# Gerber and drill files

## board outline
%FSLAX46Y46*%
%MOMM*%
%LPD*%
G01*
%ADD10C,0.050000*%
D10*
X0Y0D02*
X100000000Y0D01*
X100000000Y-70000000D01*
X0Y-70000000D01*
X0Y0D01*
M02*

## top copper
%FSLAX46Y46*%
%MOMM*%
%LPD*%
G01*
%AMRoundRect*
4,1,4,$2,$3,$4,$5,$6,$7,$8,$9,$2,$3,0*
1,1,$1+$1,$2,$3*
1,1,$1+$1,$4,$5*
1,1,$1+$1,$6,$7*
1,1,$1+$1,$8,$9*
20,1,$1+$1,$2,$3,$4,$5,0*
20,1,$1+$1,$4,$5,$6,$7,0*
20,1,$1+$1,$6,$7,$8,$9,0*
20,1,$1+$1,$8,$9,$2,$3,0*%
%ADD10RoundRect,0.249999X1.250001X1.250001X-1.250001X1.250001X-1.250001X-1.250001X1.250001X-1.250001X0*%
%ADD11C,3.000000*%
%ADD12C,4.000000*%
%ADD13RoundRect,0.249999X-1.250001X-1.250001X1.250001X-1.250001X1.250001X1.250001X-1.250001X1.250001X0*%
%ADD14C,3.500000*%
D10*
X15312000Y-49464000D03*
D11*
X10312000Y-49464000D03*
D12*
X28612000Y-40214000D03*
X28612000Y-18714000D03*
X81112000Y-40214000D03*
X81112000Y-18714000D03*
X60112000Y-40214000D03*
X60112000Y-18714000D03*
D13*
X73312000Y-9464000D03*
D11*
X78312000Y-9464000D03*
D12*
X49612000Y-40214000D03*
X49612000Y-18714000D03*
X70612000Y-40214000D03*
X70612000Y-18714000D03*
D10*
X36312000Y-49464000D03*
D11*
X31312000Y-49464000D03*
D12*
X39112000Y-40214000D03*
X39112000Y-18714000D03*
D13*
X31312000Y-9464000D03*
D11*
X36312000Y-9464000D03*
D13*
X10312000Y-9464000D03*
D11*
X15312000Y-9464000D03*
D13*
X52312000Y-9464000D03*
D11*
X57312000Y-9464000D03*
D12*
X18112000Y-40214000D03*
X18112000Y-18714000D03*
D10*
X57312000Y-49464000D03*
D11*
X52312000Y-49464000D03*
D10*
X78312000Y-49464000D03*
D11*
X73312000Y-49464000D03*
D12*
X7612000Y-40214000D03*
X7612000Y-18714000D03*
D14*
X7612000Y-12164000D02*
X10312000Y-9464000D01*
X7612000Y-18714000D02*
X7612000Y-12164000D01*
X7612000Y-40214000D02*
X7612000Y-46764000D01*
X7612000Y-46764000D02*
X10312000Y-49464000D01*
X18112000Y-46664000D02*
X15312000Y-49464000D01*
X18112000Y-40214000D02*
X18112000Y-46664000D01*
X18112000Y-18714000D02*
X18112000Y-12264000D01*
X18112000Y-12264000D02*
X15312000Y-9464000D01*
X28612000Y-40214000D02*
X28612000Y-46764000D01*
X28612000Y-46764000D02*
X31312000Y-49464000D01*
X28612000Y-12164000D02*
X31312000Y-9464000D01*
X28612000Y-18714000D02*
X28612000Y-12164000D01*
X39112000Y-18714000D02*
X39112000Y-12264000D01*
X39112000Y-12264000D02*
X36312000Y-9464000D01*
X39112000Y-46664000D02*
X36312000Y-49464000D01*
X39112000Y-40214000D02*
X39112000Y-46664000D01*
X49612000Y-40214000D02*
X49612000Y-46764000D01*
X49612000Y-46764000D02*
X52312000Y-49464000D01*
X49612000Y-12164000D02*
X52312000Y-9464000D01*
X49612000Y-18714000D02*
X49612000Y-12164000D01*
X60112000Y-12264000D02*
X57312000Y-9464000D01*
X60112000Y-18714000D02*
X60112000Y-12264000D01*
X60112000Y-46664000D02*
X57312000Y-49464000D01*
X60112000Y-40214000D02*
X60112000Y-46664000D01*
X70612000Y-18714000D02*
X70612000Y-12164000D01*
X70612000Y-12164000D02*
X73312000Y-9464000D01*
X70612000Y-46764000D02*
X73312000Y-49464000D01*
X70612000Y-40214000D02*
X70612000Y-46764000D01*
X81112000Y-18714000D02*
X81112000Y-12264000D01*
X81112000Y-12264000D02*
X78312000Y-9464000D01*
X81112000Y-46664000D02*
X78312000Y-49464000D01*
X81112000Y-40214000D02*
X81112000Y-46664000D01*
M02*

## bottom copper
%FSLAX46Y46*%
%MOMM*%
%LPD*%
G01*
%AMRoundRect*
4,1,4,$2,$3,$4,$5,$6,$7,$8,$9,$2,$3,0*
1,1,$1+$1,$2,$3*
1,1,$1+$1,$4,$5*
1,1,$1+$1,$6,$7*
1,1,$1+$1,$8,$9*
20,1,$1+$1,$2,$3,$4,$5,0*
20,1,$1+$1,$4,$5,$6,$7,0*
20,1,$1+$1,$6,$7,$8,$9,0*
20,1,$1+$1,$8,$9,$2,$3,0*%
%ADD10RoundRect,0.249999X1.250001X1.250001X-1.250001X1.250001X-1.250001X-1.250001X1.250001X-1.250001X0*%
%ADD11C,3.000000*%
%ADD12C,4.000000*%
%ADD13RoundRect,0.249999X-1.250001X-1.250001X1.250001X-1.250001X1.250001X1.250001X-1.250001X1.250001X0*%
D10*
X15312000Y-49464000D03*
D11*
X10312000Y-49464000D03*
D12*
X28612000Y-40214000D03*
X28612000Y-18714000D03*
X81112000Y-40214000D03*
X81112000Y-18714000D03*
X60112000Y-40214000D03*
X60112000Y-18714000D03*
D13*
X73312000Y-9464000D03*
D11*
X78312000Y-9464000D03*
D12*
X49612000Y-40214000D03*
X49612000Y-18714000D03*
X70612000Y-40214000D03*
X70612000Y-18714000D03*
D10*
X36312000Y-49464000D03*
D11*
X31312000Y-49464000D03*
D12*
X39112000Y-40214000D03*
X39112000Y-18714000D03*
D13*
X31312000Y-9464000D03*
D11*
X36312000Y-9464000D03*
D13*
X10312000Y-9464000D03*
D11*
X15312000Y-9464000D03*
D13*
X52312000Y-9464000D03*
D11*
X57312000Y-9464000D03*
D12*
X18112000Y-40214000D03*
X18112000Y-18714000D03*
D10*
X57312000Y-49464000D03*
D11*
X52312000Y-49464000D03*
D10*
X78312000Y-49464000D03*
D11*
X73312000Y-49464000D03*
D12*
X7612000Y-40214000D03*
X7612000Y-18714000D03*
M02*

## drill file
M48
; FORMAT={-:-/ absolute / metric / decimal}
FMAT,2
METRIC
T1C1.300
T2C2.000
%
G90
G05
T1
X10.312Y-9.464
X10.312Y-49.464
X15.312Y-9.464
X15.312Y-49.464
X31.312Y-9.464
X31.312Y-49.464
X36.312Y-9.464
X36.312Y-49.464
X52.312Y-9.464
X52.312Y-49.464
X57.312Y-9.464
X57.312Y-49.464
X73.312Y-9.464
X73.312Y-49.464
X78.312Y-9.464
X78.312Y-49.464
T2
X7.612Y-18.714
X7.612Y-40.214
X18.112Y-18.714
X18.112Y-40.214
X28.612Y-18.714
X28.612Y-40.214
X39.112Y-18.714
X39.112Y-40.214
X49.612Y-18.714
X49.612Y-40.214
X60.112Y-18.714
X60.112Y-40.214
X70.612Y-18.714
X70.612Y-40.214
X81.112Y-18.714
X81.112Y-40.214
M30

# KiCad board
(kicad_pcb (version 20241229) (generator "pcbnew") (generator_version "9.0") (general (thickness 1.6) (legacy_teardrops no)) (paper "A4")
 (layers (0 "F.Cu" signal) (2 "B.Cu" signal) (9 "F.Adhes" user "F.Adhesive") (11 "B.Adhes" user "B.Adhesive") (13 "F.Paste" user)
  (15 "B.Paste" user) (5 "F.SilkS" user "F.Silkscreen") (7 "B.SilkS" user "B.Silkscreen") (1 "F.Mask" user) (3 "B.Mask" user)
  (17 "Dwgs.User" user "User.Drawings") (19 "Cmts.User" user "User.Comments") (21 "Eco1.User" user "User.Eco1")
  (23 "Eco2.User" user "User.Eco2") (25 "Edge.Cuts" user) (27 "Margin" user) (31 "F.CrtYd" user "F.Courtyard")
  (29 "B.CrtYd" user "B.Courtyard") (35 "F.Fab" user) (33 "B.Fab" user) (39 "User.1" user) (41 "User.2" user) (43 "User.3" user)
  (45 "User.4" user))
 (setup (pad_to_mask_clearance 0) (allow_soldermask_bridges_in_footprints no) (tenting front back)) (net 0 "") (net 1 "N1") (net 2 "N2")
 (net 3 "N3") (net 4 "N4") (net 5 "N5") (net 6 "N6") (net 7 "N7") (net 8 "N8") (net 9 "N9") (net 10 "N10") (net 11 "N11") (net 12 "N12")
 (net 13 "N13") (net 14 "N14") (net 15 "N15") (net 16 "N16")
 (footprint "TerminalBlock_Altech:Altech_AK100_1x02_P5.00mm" (layer "F.Cu") (at 15.312 49.464 180)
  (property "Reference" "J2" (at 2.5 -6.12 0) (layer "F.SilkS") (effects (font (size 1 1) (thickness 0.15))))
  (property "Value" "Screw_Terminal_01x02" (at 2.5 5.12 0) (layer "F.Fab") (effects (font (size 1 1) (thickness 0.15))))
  (pad "1" thru_hole roundrect (at 0 0 180) (size 3 3) (drill 1.3) (layers "*.Cu" "*.Mask") (remove_unused_layers no)
   (roundrect_rratio 0.083333) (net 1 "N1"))
  (pad "2" thru_hole circle (at 5 0 180) (size 3 3) (drill 1.3) (layers "*.Cu" "*.Mask") (remove_unused_layers no) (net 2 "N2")))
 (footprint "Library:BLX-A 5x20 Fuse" (layer "F.Cu") (at 28.612 29.464 90)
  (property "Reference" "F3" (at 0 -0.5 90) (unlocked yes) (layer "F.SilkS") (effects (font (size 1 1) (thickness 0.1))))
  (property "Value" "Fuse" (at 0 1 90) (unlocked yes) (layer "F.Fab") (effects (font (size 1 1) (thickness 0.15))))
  (pad "1" thru_hole circle (at -10.75 0 90) (size 4 4) (drill 2) (layers "*.Cu" "*.Mask") (remove_unused_layers no) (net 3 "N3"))
  (pad "2" thru_hole circle (at 10.75 0 90) (size 4 4) (drill 2) (layers "*.Cu" "*.Mask") (remove_unused_layers no) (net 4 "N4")))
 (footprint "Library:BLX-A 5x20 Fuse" (layer "F.Cu") (at 81.112 29.464 90)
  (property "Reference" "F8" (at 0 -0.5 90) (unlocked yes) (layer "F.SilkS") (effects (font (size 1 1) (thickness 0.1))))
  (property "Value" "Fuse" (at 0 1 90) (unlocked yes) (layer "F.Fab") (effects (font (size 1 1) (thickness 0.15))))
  (pad "1" thru_hole circle (at -10.75 0 90) (size 4 4) (drill 2) (layers "*.Cu" "*.Mask") (remove_unused_layers no) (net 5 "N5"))
  (pad "2" thru_hole circle (at 10.75 0 90) (size 4 4) (drill 2) (layers "*.Cu" "*.Mask") (remove_unused_layers no) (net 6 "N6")))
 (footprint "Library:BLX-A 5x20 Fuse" (layer "F.Cu") (at 60.112 29.464 90)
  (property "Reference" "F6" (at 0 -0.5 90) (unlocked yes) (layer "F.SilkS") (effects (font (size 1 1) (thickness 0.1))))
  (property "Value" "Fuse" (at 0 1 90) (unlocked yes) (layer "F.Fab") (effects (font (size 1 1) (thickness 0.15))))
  (pad "1" thru_hole circle (at -10.75 0 90) (size 4 4) (drill 2) (layers "*.Cu" "*.Mask") (remove_unused_layers no) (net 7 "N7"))
  (pad "2" thru_hole circle (at 10.75 0 90) (size 4 4) (drill 2) (layers "*.Cu" "*.Mask") (remove_unused_layers no) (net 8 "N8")))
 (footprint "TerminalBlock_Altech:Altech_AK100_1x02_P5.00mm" (layer "F.Cu") (at 73.312 9.464)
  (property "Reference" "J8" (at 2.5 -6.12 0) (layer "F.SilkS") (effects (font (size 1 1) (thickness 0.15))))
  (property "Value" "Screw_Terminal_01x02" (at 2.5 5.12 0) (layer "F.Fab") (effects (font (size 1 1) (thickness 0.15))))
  (pad "1" thru_hole roundrect (at 0 0) (size 3 3) (drill 1.3) (layers "*.Cu" "*.Mask") (remove_unused_layers no)
   (roundrect_rratio 0.083333) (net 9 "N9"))
  (pad "2" thru_hole circle (at 5 0) (size 3 3) (drill 1.3) (layers "*.Cu" "*.Mask") (remove_unused_layers no) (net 6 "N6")))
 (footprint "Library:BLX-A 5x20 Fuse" (layer "F.Cu") (at 49.612 29.464 90)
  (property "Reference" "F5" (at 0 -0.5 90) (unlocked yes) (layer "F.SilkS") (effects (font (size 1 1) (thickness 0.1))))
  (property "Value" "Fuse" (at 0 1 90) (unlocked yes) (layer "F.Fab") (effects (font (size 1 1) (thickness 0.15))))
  (pad "1" thru_hole circle (at -10.75 0 90) (size 4 4) (drill 2) (layers "*.Cu" "*.Mask") (remove_unused_layers no) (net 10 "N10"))
  (pad "2" thru_hole circle (at 10.75 0 90) (size 4 4) (drill 2) (layers "*.Cu" "*.Mask") (remove_unused_layers no) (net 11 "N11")))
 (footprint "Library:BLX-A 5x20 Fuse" (layer "F.Cu") (at 70.612 29.464 90)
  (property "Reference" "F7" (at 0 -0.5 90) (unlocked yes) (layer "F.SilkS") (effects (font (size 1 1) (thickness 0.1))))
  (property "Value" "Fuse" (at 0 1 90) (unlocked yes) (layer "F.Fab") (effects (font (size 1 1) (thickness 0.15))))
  (pad "1" thru_hole circle (at -10.75 0 90) (size 4 4) (drill 2) (layers "*.Cu" "*.Mask") (remove_unused_layers no) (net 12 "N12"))
  (pad "2" thru_hole circle (at 10.75 0 90) (size 4 4) (drill 2) (layers "*.Cu" "*.Mask") (remove_unused_layers no) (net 9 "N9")))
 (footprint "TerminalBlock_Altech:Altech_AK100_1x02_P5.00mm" (layer "F.Cu") (at 36.312 49.464 180)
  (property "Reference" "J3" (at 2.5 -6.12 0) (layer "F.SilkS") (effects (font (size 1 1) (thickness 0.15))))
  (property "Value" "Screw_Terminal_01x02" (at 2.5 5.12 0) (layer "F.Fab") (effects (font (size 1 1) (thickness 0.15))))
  (pad "1" thru_hole roundrect (at 0 0 180) (size 3 3) (drill 1.3) (layers "*.Cu" "*.Mask") (remove_unused_layers no)
   (roundrect_rratio 0.083333) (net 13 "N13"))
  (pad "2" thru_hole circle (at 5 0 180) (size 3 3) (drill 1.3) (layers "*.Cu" "*.Mask") (remove_unused_layers no) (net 3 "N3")))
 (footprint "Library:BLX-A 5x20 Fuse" (layer "F.Cu") (at 39.112 29.464 90)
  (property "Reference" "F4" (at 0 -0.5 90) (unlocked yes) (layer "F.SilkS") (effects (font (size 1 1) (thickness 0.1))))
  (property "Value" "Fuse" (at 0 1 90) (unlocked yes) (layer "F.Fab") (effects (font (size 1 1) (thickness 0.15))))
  (pad "1" thru_hole circle (at -10.75 0 90) (size 4 4) (drill 2) (layers "*.Cu" "*.Mask") (remove_unused_layers no) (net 13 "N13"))
  (pad "2" thru_hole circle (at 10.75 0 90) (size 4 4) (drill 2) (layers "*.Cu" "*.Mask") (remove_unused_layers no) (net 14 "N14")))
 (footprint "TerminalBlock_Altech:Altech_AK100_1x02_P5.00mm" (layer "F.Cu") (at 31.312 9.464)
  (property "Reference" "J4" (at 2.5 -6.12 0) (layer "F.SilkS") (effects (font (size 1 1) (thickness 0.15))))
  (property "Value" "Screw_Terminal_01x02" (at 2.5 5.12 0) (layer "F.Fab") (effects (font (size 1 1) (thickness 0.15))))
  (pad "1" thru_hole roundrect (at 0 0) (size 3 3) (drill 1.3) (layers "*.Cu" "*.Mask") (remove_unused_layers no)
   (roundrect_rratio 0.083333) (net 4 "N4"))
  (pad "2" thru_hole circle (at 5 0) (size 3 3) (drill 1.3) (layers "*.Cu" "*.Mask") (remove_unused_layers no) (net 14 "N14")))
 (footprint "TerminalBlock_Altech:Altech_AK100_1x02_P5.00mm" (layer "F.Cu") (at 10.312 9.464)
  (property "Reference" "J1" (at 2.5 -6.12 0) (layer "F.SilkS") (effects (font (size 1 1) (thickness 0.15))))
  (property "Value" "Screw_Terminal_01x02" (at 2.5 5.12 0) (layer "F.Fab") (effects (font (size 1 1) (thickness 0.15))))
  (pad "1" thru_hole roundrect (at 0 0) (size 3 3) (drill 1.3) (layers "*.Cu" "*.Mask") (remove_unused_layers no)
   (roundrect_rratio 0.083333) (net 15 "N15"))
  (pad "2" thru_hole circle (at 5 0) (size 3 3) (drill 1.3) (layers "*.Cu" "*.Mask") (remove_unused_layers no) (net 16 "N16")))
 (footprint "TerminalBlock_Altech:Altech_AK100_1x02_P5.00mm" (layer "F.Cu") (at 52.312 9.464)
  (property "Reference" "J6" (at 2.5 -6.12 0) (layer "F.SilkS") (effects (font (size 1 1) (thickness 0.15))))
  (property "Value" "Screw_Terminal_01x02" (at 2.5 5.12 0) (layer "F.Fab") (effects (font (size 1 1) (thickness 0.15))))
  (pad "1" thru_hole roundrect (at 0 0) (size 3 3) (drill 1.3) (layers "*.Cu" "*.Mask") (remove_unused_layers no)
   (roundrect_rratio 0.083333) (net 11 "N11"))
  (pad "2" thru_hole circle (at 5 0) (size 3 3) (drill 1.3) (layers "*.Cu" "*.Mask") (remove_unused_layers no) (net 8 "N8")))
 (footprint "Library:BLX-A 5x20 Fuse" (layer "F.Cu") (at 18.112 29.464 90)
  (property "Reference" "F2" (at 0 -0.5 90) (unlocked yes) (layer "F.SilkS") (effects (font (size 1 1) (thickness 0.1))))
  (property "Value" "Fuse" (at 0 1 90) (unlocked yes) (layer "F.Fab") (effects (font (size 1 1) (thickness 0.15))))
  (pad "1" thru_hole circle (at -10.75 0 90) (size 4 4) (drill 2) (layers "*.Cu" "*.Mask") (remove_unused_layers no) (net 1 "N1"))
  (pad "2" thru_hole circle (at 10.75 0 90) (size 4 4) (drill 2) (layers "*.Cu" "*.Mask") (remove_unused_layers no) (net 16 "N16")))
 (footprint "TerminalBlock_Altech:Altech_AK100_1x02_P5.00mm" (layer "F.Cu") (at 57.312 49.464 180)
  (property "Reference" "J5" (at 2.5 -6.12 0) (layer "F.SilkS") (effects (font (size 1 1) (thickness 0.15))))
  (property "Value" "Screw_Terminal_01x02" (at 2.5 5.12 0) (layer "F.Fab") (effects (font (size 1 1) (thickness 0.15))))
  (pad "1" thru_hole roundrect (at 0 0 180) (size 3 3) (drill 1.3) (layers "*.Cu" "*.Mask") (remove_unused_layers no)
   (roundrect_rratio 0.083333) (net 7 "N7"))
  (pad "2" thru_hole circle (at 5 0 180) (size 3 3) (drill 1.3) (layers "*.Cu" "*.Mask") (remove_unused_layers no) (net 10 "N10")))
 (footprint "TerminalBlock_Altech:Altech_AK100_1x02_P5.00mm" (layer "F.Cu") (at 78.312 49.464 180)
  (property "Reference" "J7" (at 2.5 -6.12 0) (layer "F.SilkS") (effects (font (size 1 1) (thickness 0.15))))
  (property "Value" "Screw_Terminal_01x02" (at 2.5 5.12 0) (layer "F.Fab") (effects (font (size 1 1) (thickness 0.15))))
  (pad "1" thru_hole roundrect (at 0 0 180) (size 3 3) (drill 1.3) (layers "*.Cu" "*.Mask") (remove_unused_layers no)
   (roundrect_rratio 0.083333) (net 5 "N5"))
  (pad "2" thru_hole circle (at 5 0 180) (size 3 3) (drill 1.3) (layers "*.Cu" "*.Mask") (remove_unused_layers no) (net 12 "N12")))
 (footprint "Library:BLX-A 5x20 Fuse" (layer "F.Cu") (at 7.612 29.464 90)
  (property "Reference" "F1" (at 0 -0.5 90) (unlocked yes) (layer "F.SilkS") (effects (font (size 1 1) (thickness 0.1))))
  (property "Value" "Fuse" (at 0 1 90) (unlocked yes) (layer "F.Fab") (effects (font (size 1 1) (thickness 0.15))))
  (pad "1" thru_hole circle (at -10.75 0 90) (size 4 4) (drill 2) (layers "*.Cu" "*.Mask") (remove_unused_layers no) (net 2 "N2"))
  (pad "2" thru_hole circle (at 10.75 0 90) (size 4 4) (drill 2) (layers "*.Cu" "*.Mask") (remove_unused_layers no) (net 15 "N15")))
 (gr_rect (start 0 0) (end 100 70) (stroke (width 0.05) (type solid)) (fill no) (layer "Edge.Cuts"))
 (segment (start 7.612 12.164) (end 10.312 9.464) (width 3.5) (layer "F.Cu") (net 15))
 (segment (start 7.612 18.714) (end 7.612 12.164) (width 3.5) (layer "F.Cu") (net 15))
 (segment (start 7.612 40.214) (end 7.612 46.764) (width 3.5) (layer "F.Cu") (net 2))
 (segment (start 7.612 46.764) (end 10.312 49.464) (width 3.5) (layer "F.Cu") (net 2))
 (segment (start 18.112 46.664) (end 15.312 49.464) (width 3.5) (layer "F.Cu") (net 1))
 (segment (start 18.112 40.214) (end 18.112 46.664) (width 3.5) (layer "F.Cu") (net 1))
 (segment (start 18.112 18.714) (end 18.112 12.264) (width 3.5) (layer "F.Cu") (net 16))
 (segment (start 18.112 12.264) (end 15.312 9.464) (width 3.5) (layer "F.Cu") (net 16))
 (segment (start 28.612 40.214) (end 28.612 46.764) (width 3.5) (layer "F.Cu") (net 3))
 (segment (start 28.612 46.764) (end 31.312 49.464) (width 3.5) (layer "F.Cu") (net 3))
 (segment (start 28.612 12.164) (end 31.312 9.464) (width 3.5) (layer "F.Cu") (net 4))
 (segment (start 28.612 18.714) (end 28.612 12.164) (width 3.5) (layer "F.Cu") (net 4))
 (segment (start 39.112 18.714) (end 39.112 12.264) (width 3.5) (layer "F.Cu") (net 14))
 (segment (start 39.112 12.264) (end 36.312 9.464) (width 3.5) (layer "F.Cu") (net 14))
 (segment (start 39.112 46.664) (end 36.312 49.464) (width 3.5) (layer "F.Cu") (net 13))
 (segment (start 39.112 40.214) (end 39.112 46.664) (width 3.5) (layer "F.Cu") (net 13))
 (segment (start 49.612 40.214) (end 49.612 46.764) (width 3.5) (layer "F.Cu") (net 10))
 (segment (start 49.612 46.764) (end 52.312 49.464) (width 3.5) (layer "F.Cu") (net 10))
 (segment (start 49.612 12.164) (end 52.312 9.464) (width 3.5) (layer "F.Cu") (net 11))
 (segment (start 49.612 18.714) (end 49.612 12.164) (width 3.5) (layer "F.Cu") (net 11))
 (segment (start 60.112 12.264) (end 57.312 9.464) (width 3.5) (layer "F.Cu") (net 8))
 (segment (start 60.112 18.714) (end 60.112 12.264) (width 3.5) (layer "F.Cu") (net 8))
 (segment (start 60.112 46.664) (end 57.312 49.464) (width 3.5) (layer "F.Cu") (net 7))
 (segment (start 60.112 40.214) (end 60.112 46.664) (width 3.5) (layer "F.Cu") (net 7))
 (segment (start 70.612 18.714) (end 70.612 12.164) (width 3.5) (layer "F.Cu") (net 9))
 (segment (start 70.612 12.164) (end 73.312 9.464) (width 3.5) (layer "F.Cu") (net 9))
 (segment (start 70.612 46.764) (end 73.312 49.464) (width 3.5) (layer "F.Cu") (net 12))
 (segment (start 70.612 40.214) (end 70.612 46.764) (width 3.5) (layer "F.Cu") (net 12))
 (segment (start 81.112 18.714) (end 81.112 12.264) (width 3.5) (layer "F.Cu") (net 6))
 (segment (start 81.112 12.264) (end 78.312 9.464) (width 3.5) (layer "F.Cu") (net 6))
 (segment (start 81.112 46.664) (end 78.312 49.464) (width 3.5) (layer "F.Cu") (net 5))
 (segment (start 81.112 40.214) (end 81.112 46.664) (width 3.5) (layer "F.Cu") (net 5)))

